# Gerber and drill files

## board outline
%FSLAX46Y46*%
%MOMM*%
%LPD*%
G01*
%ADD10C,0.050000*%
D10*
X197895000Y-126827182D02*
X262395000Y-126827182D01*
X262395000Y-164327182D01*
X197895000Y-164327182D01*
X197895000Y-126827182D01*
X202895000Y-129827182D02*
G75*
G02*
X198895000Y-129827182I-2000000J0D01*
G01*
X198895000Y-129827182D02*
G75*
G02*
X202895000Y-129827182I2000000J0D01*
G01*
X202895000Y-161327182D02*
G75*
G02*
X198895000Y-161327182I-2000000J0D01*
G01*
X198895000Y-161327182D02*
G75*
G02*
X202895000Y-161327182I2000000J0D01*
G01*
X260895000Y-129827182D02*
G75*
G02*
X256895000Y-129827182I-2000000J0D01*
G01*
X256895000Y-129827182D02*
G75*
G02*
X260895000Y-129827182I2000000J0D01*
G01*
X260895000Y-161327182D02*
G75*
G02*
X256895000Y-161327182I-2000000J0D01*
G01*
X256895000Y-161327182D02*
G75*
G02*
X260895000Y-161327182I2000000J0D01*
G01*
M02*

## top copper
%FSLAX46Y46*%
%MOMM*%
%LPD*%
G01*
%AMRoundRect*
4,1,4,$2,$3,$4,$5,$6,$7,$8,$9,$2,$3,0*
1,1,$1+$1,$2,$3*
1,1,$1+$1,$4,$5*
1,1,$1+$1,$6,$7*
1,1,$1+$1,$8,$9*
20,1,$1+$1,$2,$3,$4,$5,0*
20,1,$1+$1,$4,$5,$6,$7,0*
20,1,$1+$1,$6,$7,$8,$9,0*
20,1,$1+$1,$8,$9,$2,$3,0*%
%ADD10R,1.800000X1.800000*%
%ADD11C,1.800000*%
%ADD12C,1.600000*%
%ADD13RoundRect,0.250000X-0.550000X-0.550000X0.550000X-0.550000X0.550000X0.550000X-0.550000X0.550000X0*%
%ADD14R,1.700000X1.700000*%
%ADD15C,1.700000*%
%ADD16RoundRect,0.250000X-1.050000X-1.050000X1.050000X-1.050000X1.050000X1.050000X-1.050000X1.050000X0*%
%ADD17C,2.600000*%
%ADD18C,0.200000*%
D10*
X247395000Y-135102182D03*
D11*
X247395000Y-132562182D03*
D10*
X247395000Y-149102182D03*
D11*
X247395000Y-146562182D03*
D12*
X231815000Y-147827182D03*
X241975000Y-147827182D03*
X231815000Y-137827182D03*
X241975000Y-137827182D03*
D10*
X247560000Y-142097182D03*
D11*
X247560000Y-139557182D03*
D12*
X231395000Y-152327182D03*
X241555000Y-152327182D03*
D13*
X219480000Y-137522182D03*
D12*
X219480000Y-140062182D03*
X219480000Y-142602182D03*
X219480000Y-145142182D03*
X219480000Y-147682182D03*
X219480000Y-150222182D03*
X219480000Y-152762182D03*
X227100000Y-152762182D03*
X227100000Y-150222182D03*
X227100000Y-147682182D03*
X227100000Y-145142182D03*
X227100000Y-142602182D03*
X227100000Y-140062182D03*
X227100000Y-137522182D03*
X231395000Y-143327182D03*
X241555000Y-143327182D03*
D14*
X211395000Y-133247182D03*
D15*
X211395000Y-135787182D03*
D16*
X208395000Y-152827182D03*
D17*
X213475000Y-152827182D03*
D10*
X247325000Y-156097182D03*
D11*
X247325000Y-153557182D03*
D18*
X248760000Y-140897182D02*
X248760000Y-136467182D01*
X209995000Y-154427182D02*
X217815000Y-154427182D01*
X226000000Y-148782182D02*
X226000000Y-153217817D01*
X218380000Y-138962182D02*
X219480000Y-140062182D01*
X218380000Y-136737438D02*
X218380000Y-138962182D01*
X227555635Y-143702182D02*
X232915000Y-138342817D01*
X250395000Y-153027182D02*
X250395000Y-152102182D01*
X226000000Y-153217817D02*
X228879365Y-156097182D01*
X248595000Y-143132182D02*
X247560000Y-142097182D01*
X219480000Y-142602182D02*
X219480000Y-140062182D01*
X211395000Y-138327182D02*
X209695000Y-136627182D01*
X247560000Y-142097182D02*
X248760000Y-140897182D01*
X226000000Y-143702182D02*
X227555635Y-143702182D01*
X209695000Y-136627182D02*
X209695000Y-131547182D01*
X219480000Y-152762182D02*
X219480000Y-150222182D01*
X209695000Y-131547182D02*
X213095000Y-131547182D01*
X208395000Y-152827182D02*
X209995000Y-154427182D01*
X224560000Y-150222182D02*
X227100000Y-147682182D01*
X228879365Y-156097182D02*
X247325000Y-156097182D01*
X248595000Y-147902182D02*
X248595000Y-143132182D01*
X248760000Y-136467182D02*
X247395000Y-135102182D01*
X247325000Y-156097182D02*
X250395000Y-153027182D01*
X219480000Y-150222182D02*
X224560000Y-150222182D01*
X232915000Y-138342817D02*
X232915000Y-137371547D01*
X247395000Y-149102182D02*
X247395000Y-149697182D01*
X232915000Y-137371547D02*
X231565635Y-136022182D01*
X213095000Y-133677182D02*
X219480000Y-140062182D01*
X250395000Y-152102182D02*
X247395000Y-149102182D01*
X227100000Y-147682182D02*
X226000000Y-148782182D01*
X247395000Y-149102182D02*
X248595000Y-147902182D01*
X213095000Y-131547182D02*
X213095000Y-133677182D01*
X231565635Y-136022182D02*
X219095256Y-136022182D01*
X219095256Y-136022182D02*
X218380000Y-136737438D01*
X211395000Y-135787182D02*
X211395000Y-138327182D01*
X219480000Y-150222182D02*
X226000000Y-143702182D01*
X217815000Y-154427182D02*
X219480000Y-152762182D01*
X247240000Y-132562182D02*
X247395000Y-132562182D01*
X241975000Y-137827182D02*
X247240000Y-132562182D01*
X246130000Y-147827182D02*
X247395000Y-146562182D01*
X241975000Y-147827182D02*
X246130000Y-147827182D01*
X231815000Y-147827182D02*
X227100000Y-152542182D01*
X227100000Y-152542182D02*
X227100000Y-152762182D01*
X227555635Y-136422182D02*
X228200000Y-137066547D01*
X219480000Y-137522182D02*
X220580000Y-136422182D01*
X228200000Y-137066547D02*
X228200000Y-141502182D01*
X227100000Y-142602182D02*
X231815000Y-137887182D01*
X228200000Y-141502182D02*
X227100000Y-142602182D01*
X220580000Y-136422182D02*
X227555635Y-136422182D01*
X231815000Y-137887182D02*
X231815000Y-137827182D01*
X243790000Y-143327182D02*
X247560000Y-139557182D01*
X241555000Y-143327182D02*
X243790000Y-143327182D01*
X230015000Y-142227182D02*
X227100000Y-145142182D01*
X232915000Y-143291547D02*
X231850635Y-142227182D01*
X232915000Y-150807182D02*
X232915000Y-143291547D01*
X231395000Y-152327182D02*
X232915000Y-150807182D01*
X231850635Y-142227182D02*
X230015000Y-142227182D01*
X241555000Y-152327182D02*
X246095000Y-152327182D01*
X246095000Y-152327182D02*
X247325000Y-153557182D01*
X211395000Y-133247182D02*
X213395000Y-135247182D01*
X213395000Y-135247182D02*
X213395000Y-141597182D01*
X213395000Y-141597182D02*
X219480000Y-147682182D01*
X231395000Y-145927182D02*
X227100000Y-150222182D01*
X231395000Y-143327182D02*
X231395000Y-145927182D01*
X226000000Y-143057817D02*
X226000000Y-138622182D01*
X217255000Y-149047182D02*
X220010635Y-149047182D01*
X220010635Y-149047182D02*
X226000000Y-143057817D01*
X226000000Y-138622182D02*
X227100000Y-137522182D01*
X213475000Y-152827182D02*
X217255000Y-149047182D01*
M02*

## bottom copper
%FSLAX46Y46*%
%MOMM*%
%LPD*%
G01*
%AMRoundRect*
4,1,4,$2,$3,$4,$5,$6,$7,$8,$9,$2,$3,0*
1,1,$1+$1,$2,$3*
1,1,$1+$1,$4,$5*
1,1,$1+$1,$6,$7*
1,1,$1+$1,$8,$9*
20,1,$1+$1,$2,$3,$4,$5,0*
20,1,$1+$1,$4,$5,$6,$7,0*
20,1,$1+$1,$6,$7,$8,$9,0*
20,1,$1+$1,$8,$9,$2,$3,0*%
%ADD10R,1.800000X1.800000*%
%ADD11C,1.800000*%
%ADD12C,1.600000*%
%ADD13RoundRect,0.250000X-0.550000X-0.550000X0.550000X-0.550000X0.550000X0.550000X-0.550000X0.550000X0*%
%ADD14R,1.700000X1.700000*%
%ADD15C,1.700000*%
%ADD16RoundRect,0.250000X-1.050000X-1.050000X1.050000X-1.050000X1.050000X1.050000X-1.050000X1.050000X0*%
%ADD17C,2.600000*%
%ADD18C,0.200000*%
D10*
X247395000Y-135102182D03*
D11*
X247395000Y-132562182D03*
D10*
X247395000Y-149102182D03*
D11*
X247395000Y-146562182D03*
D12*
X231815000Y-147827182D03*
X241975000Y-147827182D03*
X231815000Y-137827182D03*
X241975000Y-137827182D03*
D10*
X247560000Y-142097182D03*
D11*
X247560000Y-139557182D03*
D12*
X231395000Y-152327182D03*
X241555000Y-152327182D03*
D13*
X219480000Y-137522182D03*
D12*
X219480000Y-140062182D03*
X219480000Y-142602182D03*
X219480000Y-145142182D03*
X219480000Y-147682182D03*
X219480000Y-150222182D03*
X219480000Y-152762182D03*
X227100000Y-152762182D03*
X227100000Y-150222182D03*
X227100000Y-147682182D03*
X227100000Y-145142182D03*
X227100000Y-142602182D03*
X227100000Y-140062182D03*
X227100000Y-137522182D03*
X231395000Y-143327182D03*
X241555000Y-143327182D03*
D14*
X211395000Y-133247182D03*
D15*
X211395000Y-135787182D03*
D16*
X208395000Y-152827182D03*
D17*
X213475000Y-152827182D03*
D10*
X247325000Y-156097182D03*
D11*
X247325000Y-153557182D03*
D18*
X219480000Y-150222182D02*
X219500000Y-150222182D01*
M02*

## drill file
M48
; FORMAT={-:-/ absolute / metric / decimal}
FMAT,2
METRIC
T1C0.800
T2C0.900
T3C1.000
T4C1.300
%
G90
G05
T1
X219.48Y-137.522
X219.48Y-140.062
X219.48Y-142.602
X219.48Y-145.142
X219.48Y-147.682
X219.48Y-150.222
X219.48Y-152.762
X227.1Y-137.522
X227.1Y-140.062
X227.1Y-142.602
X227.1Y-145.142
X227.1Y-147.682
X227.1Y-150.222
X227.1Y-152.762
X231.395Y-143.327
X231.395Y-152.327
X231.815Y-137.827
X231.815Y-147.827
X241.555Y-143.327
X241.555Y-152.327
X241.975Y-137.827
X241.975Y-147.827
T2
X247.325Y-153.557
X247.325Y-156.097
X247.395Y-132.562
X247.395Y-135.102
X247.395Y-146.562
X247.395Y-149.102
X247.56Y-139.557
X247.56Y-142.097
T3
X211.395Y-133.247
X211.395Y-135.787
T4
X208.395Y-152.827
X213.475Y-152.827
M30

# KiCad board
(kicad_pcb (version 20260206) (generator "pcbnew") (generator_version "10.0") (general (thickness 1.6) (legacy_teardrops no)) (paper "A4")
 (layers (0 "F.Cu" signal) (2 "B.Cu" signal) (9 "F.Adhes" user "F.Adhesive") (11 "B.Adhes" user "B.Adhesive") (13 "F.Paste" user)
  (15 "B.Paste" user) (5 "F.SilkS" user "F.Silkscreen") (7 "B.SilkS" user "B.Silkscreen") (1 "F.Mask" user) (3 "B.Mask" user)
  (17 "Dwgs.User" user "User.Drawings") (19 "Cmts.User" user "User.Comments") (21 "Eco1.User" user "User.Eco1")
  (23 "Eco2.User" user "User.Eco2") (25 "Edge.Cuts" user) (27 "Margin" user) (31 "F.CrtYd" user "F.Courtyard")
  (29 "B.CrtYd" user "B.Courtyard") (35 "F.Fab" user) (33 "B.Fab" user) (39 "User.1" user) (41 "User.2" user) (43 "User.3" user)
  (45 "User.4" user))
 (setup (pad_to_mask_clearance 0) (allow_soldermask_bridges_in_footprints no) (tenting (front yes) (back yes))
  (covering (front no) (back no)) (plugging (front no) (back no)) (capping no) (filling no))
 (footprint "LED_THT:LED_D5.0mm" (layer "F.Cu") (at 247.395 135.102182 90)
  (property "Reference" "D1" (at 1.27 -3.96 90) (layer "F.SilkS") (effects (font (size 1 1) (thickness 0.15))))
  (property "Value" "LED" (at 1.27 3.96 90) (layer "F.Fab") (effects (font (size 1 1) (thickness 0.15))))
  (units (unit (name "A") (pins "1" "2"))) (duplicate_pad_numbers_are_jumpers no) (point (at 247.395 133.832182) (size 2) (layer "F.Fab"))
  (pad "1" thru_hole rect (at 0 0 90) (size 1.8 1.8) (drill 0.9) (layers "*.Cu" "*.Mask") (remove_unused_layers no) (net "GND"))
  (pad "2" thru_hole circle (at 2.54 0 90) (size 1.8 1.8) (drill 0.9) (layers "*.Cu" "*.Mask") (remove_unused_layers no) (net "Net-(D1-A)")))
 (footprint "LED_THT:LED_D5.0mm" (layer "F.Cu") (at 247.395 149.102182 90)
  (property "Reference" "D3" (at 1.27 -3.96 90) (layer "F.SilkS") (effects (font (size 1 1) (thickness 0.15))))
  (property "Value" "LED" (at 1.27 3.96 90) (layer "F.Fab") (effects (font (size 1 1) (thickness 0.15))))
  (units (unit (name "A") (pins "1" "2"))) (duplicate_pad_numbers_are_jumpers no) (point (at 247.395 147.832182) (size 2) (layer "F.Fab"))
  (pad "1" thru_hole rect (at 0 0 90) (size 1.8 1.8) (drill 0.9) (layers "*.Cu" "*.Mask") (remove_unused_layers no) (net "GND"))
  (pad "2" thru_hole circle (at 2.54 0 90) (size 1.8 1.8) (drill 0.9) (layers "*.Cu" "*.Mask") (remove_unused_layers no) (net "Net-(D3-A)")))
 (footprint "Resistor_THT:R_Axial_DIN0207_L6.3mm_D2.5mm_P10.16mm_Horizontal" (layer "F.Cu") (at 231.815 147.827182)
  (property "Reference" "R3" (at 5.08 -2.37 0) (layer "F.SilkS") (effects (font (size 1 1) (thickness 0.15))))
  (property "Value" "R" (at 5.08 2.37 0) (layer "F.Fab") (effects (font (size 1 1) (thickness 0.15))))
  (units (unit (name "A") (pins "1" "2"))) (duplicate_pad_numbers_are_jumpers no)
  (pad "1" thru_hole circle (at 0 0) (size 1.6 1.6) (drill 0.8) (layers "*.Cu" "*.Mask") (remove_unused_layers no) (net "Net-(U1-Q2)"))
  (pad "2" thru_hole circle (at 10.16 0) (size 1.6 1.6) (drill 0.8) (layers "*.Cu" "*.Mask") (remove_unused_layers no) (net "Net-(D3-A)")))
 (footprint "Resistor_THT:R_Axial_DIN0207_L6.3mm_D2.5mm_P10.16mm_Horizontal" (layer "F.Cu") (at 231.815 137.827182)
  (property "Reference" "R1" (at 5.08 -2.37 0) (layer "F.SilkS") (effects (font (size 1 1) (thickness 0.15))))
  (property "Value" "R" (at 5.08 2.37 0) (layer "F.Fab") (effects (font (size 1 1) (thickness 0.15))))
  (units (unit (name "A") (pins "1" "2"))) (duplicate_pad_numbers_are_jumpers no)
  (pad "1" thru_hole circle (at 0 0) (size 1.6 1.6) (drill 0.8) (layers "*.Cu" "*.Mask") (remove_unused_layers no) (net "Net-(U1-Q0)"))
  (pad "2" thru_hole circle (at 10.16 0) (size 1.6 1.6) (drill 0.8) (layers "*.Cu" "*.Mask") (remove_unused_layers no) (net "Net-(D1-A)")))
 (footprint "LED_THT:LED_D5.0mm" (layer "F.Cu") (at 247.56 142.097182 90)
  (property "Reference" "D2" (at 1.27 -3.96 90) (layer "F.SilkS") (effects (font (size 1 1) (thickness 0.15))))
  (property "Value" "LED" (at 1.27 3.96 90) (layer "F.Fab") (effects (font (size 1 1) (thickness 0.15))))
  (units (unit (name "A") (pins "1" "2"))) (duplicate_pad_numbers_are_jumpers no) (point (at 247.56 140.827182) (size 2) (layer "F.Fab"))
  (pad "1" thru_hole rect (at 0 0 90) (size 1.8 1.8) (drill 0.9) (layers "*.Cu" "*.Mask") (remove_unused_layers no) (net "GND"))
  (pad "2" thru_hole circle (at 2.54 0 90) (size 1.8 1.8) (drill 0.9) (layers "*.Cu" "*.Mask") (remove_unused_layers no) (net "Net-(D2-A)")))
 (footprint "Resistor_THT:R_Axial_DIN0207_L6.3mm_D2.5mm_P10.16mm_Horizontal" (layer "F.Cu") (at 231.395 152.327182)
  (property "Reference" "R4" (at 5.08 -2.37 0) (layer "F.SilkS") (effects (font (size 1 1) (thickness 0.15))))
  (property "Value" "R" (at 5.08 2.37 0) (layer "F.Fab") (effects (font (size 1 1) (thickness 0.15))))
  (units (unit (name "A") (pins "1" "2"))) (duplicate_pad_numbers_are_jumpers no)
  (pad "1" thru_hole circle (at 0 0) (size 1.6 1.6) (drill 0.8) (layers "*.Cu" "*.Mask") (remove_unused_layers no) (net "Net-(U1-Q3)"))
  (pad "2" thru_hole circle (at 10.16 0) (size 1.6 1.6) (drill 0.8) (layers "*.Cu" "*.Mask") (remove_unused_layers no) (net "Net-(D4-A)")))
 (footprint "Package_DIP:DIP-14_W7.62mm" (layer "F.Cu") (at 219.48 137.522182)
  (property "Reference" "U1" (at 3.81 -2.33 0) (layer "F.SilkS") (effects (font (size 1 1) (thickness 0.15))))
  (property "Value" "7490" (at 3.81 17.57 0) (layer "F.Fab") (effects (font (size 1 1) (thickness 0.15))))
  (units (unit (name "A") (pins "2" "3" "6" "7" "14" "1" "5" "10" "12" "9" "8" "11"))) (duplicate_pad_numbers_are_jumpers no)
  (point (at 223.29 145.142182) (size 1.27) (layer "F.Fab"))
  (pad "1" thru_hole roundrect (at 0 0) (size 1.6 1.6) (drill 0.8) (layers "*.Cu" "*.Mask") (remove_unused_layers no)
   (roundrect_rratio 0.15625) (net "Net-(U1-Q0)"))
  (pad "2" thru_hole circle (at 0 2.54) (size 1.6 1.6) (drill 0.8) (layers "*.Cu" "*.Mask") (remove_unused_layers no) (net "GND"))
  (pad "3" thru_hole circle (at 0 5.08) (size 1.6 1.6) (drill 0.8) (layers "*.Cu" "*.Mask") (remove_unused_layers no) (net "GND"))
  (pad "4" thru_hole circle (at 0 7.62) (size 1.6 1.6) (drill 0.8) (layers "*.Cu" "*.Mask") (remove_unused_layers no))
  (pad "5" thru_hole circle (at 0 10.16) (size 1.6 1.6) (drill 0.8) (layers "*.Cu" "*.Mask") (remove_unused_layers no)
   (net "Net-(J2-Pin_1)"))
  (pad "6" thru_hole circle (at 0 12.7) (size 1.6 1.6) (drill 0.8) (layers "*.Cu" "*.Mask") (remove_unused_layers no) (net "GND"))
  (pad "7" thru_hole circle (at 0 15.24) (size 1.6 1.6) (drill 0.8) (layers "*.Cu" "*.Mask") (remove_unused_layers no) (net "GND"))
  (pad "8" thru_hole circle (at 7.62 15.24) (size 1.6 1.6) (drill 0.8) (layers "*.Cu" "*.Mask") (remove_unused_layers no)
   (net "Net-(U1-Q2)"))
  (pad "9" thru_hole circle (at 7.62 12.7) (size 1.6 1.6) (drill 0.8) (layers "*.Cu" "*.Mask") (remove_unused_layers no) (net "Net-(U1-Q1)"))
  (pad "10" thru_hole circle (at 7.62 10.16) (size 1.6 1.6) (drill 0.8) (layers "*.Cu" "*.Mask") (remove_unused_layers no) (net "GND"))
  (pad "11" thru_hole circle (at 7.62 7.62) (size 1.6 1.6) (drill 0.8) (layers "*.Cu" "*.Mask") (remove_unused_layers no)
   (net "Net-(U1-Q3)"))
  (pad "12" thru_hole circle (at 7.62 5.08) (size 1.6 1.6) (drill 0.8) (layers "*.Cu" "*.Mask") (remove_unused_layers no)
   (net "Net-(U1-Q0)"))
  (pad "13" thru_hole circle (at 7.62 2.54) (size 1.6 1.6) (drill 0.8) (layers "*.Cu" "*.Mask") (remove_unused_layers no))
  (pad "14" thru_hole circle (at 7.62 0) (size 1.6 1.6) (drill 0.8) (layers "*.Cu" "*.Mask") (remove_unused_layers no)
   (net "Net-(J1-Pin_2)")))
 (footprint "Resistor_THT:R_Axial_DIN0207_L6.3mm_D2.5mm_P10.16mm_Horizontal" (layer "F.Cu") (at 231.395 143.327182)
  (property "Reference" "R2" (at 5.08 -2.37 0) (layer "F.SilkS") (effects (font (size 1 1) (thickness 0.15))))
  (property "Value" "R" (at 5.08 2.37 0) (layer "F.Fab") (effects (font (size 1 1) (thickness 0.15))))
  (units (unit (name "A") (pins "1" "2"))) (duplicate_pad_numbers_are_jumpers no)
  (pad "1" thru_hole circle (at 0 0) (size 1.6 1.6) (drill 0.8) (layers "*.Cu" "*.Mask") (remove_unused_layers no) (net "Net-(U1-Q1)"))
  (pad "2" thru_hole circle (at 10.16 0) (size 1.6 1.6) (drill 0.8) (layers "*.Cu" "*.Mask") (remove_unused_layers no) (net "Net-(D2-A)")))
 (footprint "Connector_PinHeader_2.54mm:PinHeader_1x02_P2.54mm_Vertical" (layer "F.Cu") (at 211.395 133.247182)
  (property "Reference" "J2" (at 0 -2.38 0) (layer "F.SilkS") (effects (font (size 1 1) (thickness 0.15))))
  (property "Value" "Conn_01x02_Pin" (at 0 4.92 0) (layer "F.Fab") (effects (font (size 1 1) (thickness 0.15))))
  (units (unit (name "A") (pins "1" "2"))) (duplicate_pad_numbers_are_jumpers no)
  (pad "1" thru_hole rect (at 0 0) (size 1.7 1.7) (drill 1) (layers "*.Cu" "*.Mask") (remove_unused_layers no) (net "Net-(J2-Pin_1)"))
  (pad "2" thru_hole circle (at 0 2.54) (size 1.7 1.7) (drill 1) (layers "*.Cu" "*.Mask") (remove_unused_layers no) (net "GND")))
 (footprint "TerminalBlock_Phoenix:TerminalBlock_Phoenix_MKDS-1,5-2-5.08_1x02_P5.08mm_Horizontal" (layer "F.Cu") (at 208.395 152.827182)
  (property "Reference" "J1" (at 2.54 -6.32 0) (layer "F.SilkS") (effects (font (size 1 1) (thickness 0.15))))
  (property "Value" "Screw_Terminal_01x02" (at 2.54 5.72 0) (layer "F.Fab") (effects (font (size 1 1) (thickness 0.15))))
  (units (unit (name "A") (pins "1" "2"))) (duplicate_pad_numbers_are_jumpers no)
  (pad "1" thru_hole roundrect (at 0 0) (size 2.6 2.6) (drill 1.3) (layers "*.Cu" "*.Mask") (remove_unused_layers no)
   (roundrect_rratio 0.096154) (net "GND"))
  (pad "2" thru_hole circle (at 5.08 0) (size 2.6 2.6) (drill 1.3) (layers "*.Cu" "*.Mask") (remove_unused_layers no) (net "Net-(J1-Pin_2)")))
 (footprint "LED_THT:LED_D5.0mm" (layer "F.Cu") (at 247.325 156.097182 90)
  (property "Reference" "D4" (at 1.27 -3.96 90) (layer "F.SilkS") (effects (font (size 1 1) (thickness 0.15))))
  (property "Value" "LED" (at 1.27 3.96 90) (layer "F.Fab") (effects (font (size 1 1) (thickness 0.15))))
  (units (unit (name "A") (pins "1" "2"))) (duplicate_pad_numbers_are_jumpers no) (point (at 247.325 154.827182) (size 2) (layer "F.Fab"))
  (pad "1" thru_hole rect (at 0 0 90) (size 1.8 1.8) (drill 0.9) (layers "*.Cu" "*.Mask") (remove_unused_layers no) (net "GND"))
  (pad "2" thru_hole circle (at 2.54 0 90) (size 1.8 1.8) (drill 0.9) (layers "*.Cu" "*.Mask") (remove_unused_layers no) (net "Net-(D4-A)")))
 (gr_rect (start 197.895 126.827182) (end 262.395 164.327182) (stroke (width 0.05) (type default)) (fill no) (layer "Edge.Cuts"))
 (gr_circle (center 200.895 129.827182) (end 202.895 129.827182) (stroke (width 0.05) (type solid)) (fill no) (layer "Edge.Cuts"))
 (gr_circle (center 200.895 161.327182) (end 202.895 161.327182) (stroke (width 0.05) (type solid)) (fill no) (layer "Edge.Cuts"))
 (gr_circle (center 258.895 129.827182) (end 260.895 129.827182) (stroke (width 0.05) (type solid)) (fill no) (layer "Edge.Cuts"))
 (gr_circle (center 258.895 161.327182) (end 260.895 161.327182) (stroke (width 0.05) (type solid)) (fill no) (layer "Edge.Cuts"))
 (segment (start 248.76 140.897182) (end 248.76 136.467182) (width 0.2) (layer "F.Cu") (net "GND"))
 (segment (start 209.995 154.427182) (end 217.815 154.427182) (width 0.2) (layer "F.Cu") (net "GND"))
 (segment (start 226 148.782182) (end 226 153.217817) (width 0.2) (layer "F.Cu") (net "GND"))
 (segment (start 218.38 138.962182) (end 219.48 140.062182) (width 0.2) (layer "F.Cu") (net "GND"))
 (segment (start 218.38 136.737438) (end 218.38 138.962182) (width 0.2) (layer "F.Cu") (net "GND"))
 (segment (start 227.555635 143.702182) (end 232.915 138.342817) (width 0.2) (layer "F.Cu") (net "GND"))
 (segment (start 250.395 153.027182) (end 250.395 152.102182) (width 0.2) (layer "F.Cu") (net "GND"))
 (segment (start 226 153.217817) (end 228.879365 156.097182) (width 0.2) (layer "F.Cu") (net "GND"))
 (segment (start 248.595 143.132182) (end 247.56 142.097182) (width 0.2) (layer "F.Cu") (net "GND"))
 (segment (start 219.48 142.602182) (end 219.48 140.062182) (width 0.2) (layer "F.Cu") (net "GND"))
 (segment (start 211.395 138.327182) (end 209.695 136.627182) (width 0.2) (layer "F.Cu") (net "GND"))
 (segment (start 247.56 142.097182) (end 248.76 140.897182) (width 0.2) (layer "F.Cu") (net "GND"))
 (segment (start 226 143.702182) (end 227.555635 143.702182) (width 0.2) (layer "F.Cu") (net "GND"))
 (segment (start 209.695 136.627182) (end 209.695 131.547182) (width 0.2) (layer "F.Cu") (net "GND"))
 (segment (start 219.48 152.762182) (end 219.48 150.222182) (width 0.2) (layer "F.Cu") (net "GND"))
 (segment (start 209.695 131.547182) (end 213.095 131.547182) (width 0.2) (layer "F.Cu") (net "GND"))
 (segment (start 208.395 152.827182) (end 209.995 154.427182) (width 0.2) (layer "F.Cu") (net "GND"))
 (segment (start 224.56 150.222182) (end 227.1 147.682182) (width 0.2) (layer "F.Cu") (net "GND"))
 (segment (start 228.879365 156.097182) (end 247.325 156.097182) (width 0.2) (layer "F.Cu") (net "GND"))
 (segment (start 248.595 147.902182) (end 248.595 143.132182) (width 0.2) (layer "F.Cu") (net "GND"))
 (segment (start 248.76 136.467182) (end 247.395 135.102182) (width 0.2) (layer "F.Cu") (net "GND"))
 (segment (start 247.325 156.097182) (end 250.395 153.027182) (width 0.2) (layer "F.Cu") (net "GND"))
 (segment (start 219.48 150.222182) (end 224.56 150.222182) (width 0.2) (layer "F.Cu") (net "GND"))
 (segment (start 232.915 138.342817) (end 232.915 137.371547) (width 0.2) (layer "F.Cu") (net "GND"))
 (segment (start 247.395 149.102182) (end 247.395 149.697182) (width 0.2) (layer "F.Cu") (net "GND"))
 (segment (start 232.915 137.371547) (end 231.565635 136.022182) (width 0.2) (layer "F.Cu") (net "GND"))
 (segment (start 213.095 133.677182) (end 219.48 140.062182) (width 0.2) (layer "F.Cu") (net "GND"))
 (segment (start 250.395 152.102182) (end 247.395 149.102182) (width 0.2) (layer "F.Cu") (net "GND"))
 (segment (start 227.1 147.682182) (end 226 148.782182) (width 0.2) (layer "F.Cu") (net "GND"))
 (segment (start 247.395 149.102182) (end 248.595 147.902182) (width 0.2) (layer "F.Cu") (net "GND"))
 (segment (start 213.095 131.547182) (end 213.095 133.677182) (width 0.2) (layer "F.Cu") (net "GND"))
 (segment (start 231.565635 136.022182) (end 219.095256 136.022182) (width 0.2) (layer "F.Cu") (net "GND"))
 (segment (start 219.095256 136.022182) (end 218.38 136.737438) (width 0.2) (layer "F.Cu") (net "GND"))
 (segment (start 211.395 135.787182) (end 211.395 138.327182) (width 0.2) (layer "F.Cu") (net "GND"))
 (segment (start 219.48 150.222182) (end 226 143.702182) (width 0.2) (layer "F.Cu") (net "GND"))
 (segment (start 217.815 154.427182) (end 219.48 152.762182) (width 0.2) (layer "F.Cu") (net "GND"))
 (segment (start 219.48 150.222182) (end 219.5 150.222182) (width 0.2) (layer "B.Cu") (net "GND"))
 (segment (start 247.24 132.562182) (end 247.395 132.562182) (width 0.2) (layer "F.Cu") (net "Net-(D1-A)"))
 (segment (start 241.975 137.827182) (end 247.24 132.562182) (width 0.2) (layer "F.Cu") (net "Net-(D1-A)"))
 (segment (start 246.13 147.827182) (end 247.395 146.562182) (width 0.2) (layer "F.Cu") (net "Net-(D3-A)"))
 (segment (start 241.975 147.827182) (end 246.13 147.827182) (width 0.2) (layer "F.Cu") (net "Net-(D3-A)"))
 (segment (start 231.815 147.827182) (end 227.1 152.542182) (width 0.2) (layer "F.Cu") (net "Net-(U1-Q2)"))
 (segment (start 227.1 152.542182) (end 227.1 152.762182) (width 0.2) (layer "F.Cu") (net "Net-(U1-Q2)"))
 (segment (start 227.555635 136.422182) (end 228.2 137.066547) (width 0.2) (layer "F.Cu") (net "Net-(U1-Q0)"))
 (segment (start 219.48 137.522182) (end 220.58 136.422182) (width 0.2) (layer "F.Cu") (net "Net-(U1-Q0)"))
 (segment (start 228.2 137.066547) (end 228.2 141.502182) (width 0.2) (layer "F.Cu") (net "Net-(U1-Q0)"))
 (segment (start 227.1 142.602182) (end 231.815 137.887182) (width 0.2) (layer "F.Cu") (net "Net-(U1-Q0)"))
 (segment (start 228.2 141.502182) (end 227.1 142.602182) (width 0.2) (layer "F.Cu") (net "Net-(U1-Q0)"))
 (segment (start 220.58 136.422182) (end 227.555635 136.422182) (width 0.2) (layer "F.Cu") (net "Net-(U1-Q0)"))
 (segment (start 231.815 137.887182) (end 231.815 137.827182) (width 0.2) (layer "F.Cu") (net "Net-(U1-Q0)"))
 (segment (start 243.79 143.327182) (end 247.56 139.557182) (width 0.2) (layer "F.Cu") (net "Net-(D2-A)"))
 (segment (start 241.555 143.327182) (end 243.79 143.327182) (width 0.2) (layer "F.Cu") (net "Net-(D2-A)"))
 (segment (start 230.015 142.227182) (end 227.1 145.142182) (width 0.2) (layer "F.Cu") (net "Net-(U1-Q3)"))
 (segment (start 232.915 143.291547) (end 231.850635 142.227182) (width 0.2) (layer "F.Cu") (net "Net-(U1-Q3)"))
 (segment (start 232.915 150.807182) (end 232.915 143.291547) (width 0.2) (layer "F.Cu") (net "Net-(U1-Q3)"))
 (segment (start 231.395 152.327182) (end 232.915 150.807182) (width 0.2) (layer "F.Cu") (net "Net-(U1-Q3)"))
 (segment (start 231.850635 142.227182) (end 230.015 142.227182) (width 0.2) (layer "F.Cu") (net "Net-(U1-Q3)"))
 (segment (start 241.555 152.327182) (end 246.095 152.327182) (width 0.2) (layer "F.Cu") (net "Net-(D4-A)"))
 (segment (start 246.095 152.327182) (end 247.325 153.557182) (width 0.2) (layer "F.Cu") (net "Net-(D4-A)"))
 (segment (start 211.395 133.247182) (end 213.395 135.247182) (width 0.2) (layer "F.Cu") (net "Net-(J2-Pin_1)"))
 (segment (start 213.395 135.247182) (end 213.395 141.597182) (width 0.2) (layer "F.Cu") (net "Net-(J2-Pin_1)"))
 (segment (start 213.395 141.597182) (end 219.48 147.682182) (width 0.2) (layer "F.Cu") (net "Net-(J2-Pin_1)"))
 (segment (start 231.395 145.927182) (end 227.1 150.222182) (width 0.2) (layer "F.Cu") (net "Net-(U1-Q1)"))
 (segment (start 231.395 143.327182) (end 231.395 145.927182) (width 0.2) (layer "F.Cu") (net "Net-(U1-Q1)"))
 (segment (start 226 143.057817) (end 226 138.622182) (width 0.2) (layer "F.Cu") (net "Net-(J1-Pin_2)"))
 (segment (start 217.255 149.047182) (end 220.010635 149.047182) (width 0.2) (layer "F.Cu") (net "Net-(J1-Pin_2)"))
 (segment (start 220.010635 149.047182) (end 226 143.057817) (width 0.2) (layer "F.Cu") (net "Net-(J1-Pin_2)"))
 (segment (start 226 138.622182) (end 227.1 137.522182) (width 0.2) (layer "F.Cu") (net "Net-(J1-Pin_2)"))
 (segment (start 213.475 152.827182) (end 217.255 149.047182) (width 0.2) (layer "F.Cu") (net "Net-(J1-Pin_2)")))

